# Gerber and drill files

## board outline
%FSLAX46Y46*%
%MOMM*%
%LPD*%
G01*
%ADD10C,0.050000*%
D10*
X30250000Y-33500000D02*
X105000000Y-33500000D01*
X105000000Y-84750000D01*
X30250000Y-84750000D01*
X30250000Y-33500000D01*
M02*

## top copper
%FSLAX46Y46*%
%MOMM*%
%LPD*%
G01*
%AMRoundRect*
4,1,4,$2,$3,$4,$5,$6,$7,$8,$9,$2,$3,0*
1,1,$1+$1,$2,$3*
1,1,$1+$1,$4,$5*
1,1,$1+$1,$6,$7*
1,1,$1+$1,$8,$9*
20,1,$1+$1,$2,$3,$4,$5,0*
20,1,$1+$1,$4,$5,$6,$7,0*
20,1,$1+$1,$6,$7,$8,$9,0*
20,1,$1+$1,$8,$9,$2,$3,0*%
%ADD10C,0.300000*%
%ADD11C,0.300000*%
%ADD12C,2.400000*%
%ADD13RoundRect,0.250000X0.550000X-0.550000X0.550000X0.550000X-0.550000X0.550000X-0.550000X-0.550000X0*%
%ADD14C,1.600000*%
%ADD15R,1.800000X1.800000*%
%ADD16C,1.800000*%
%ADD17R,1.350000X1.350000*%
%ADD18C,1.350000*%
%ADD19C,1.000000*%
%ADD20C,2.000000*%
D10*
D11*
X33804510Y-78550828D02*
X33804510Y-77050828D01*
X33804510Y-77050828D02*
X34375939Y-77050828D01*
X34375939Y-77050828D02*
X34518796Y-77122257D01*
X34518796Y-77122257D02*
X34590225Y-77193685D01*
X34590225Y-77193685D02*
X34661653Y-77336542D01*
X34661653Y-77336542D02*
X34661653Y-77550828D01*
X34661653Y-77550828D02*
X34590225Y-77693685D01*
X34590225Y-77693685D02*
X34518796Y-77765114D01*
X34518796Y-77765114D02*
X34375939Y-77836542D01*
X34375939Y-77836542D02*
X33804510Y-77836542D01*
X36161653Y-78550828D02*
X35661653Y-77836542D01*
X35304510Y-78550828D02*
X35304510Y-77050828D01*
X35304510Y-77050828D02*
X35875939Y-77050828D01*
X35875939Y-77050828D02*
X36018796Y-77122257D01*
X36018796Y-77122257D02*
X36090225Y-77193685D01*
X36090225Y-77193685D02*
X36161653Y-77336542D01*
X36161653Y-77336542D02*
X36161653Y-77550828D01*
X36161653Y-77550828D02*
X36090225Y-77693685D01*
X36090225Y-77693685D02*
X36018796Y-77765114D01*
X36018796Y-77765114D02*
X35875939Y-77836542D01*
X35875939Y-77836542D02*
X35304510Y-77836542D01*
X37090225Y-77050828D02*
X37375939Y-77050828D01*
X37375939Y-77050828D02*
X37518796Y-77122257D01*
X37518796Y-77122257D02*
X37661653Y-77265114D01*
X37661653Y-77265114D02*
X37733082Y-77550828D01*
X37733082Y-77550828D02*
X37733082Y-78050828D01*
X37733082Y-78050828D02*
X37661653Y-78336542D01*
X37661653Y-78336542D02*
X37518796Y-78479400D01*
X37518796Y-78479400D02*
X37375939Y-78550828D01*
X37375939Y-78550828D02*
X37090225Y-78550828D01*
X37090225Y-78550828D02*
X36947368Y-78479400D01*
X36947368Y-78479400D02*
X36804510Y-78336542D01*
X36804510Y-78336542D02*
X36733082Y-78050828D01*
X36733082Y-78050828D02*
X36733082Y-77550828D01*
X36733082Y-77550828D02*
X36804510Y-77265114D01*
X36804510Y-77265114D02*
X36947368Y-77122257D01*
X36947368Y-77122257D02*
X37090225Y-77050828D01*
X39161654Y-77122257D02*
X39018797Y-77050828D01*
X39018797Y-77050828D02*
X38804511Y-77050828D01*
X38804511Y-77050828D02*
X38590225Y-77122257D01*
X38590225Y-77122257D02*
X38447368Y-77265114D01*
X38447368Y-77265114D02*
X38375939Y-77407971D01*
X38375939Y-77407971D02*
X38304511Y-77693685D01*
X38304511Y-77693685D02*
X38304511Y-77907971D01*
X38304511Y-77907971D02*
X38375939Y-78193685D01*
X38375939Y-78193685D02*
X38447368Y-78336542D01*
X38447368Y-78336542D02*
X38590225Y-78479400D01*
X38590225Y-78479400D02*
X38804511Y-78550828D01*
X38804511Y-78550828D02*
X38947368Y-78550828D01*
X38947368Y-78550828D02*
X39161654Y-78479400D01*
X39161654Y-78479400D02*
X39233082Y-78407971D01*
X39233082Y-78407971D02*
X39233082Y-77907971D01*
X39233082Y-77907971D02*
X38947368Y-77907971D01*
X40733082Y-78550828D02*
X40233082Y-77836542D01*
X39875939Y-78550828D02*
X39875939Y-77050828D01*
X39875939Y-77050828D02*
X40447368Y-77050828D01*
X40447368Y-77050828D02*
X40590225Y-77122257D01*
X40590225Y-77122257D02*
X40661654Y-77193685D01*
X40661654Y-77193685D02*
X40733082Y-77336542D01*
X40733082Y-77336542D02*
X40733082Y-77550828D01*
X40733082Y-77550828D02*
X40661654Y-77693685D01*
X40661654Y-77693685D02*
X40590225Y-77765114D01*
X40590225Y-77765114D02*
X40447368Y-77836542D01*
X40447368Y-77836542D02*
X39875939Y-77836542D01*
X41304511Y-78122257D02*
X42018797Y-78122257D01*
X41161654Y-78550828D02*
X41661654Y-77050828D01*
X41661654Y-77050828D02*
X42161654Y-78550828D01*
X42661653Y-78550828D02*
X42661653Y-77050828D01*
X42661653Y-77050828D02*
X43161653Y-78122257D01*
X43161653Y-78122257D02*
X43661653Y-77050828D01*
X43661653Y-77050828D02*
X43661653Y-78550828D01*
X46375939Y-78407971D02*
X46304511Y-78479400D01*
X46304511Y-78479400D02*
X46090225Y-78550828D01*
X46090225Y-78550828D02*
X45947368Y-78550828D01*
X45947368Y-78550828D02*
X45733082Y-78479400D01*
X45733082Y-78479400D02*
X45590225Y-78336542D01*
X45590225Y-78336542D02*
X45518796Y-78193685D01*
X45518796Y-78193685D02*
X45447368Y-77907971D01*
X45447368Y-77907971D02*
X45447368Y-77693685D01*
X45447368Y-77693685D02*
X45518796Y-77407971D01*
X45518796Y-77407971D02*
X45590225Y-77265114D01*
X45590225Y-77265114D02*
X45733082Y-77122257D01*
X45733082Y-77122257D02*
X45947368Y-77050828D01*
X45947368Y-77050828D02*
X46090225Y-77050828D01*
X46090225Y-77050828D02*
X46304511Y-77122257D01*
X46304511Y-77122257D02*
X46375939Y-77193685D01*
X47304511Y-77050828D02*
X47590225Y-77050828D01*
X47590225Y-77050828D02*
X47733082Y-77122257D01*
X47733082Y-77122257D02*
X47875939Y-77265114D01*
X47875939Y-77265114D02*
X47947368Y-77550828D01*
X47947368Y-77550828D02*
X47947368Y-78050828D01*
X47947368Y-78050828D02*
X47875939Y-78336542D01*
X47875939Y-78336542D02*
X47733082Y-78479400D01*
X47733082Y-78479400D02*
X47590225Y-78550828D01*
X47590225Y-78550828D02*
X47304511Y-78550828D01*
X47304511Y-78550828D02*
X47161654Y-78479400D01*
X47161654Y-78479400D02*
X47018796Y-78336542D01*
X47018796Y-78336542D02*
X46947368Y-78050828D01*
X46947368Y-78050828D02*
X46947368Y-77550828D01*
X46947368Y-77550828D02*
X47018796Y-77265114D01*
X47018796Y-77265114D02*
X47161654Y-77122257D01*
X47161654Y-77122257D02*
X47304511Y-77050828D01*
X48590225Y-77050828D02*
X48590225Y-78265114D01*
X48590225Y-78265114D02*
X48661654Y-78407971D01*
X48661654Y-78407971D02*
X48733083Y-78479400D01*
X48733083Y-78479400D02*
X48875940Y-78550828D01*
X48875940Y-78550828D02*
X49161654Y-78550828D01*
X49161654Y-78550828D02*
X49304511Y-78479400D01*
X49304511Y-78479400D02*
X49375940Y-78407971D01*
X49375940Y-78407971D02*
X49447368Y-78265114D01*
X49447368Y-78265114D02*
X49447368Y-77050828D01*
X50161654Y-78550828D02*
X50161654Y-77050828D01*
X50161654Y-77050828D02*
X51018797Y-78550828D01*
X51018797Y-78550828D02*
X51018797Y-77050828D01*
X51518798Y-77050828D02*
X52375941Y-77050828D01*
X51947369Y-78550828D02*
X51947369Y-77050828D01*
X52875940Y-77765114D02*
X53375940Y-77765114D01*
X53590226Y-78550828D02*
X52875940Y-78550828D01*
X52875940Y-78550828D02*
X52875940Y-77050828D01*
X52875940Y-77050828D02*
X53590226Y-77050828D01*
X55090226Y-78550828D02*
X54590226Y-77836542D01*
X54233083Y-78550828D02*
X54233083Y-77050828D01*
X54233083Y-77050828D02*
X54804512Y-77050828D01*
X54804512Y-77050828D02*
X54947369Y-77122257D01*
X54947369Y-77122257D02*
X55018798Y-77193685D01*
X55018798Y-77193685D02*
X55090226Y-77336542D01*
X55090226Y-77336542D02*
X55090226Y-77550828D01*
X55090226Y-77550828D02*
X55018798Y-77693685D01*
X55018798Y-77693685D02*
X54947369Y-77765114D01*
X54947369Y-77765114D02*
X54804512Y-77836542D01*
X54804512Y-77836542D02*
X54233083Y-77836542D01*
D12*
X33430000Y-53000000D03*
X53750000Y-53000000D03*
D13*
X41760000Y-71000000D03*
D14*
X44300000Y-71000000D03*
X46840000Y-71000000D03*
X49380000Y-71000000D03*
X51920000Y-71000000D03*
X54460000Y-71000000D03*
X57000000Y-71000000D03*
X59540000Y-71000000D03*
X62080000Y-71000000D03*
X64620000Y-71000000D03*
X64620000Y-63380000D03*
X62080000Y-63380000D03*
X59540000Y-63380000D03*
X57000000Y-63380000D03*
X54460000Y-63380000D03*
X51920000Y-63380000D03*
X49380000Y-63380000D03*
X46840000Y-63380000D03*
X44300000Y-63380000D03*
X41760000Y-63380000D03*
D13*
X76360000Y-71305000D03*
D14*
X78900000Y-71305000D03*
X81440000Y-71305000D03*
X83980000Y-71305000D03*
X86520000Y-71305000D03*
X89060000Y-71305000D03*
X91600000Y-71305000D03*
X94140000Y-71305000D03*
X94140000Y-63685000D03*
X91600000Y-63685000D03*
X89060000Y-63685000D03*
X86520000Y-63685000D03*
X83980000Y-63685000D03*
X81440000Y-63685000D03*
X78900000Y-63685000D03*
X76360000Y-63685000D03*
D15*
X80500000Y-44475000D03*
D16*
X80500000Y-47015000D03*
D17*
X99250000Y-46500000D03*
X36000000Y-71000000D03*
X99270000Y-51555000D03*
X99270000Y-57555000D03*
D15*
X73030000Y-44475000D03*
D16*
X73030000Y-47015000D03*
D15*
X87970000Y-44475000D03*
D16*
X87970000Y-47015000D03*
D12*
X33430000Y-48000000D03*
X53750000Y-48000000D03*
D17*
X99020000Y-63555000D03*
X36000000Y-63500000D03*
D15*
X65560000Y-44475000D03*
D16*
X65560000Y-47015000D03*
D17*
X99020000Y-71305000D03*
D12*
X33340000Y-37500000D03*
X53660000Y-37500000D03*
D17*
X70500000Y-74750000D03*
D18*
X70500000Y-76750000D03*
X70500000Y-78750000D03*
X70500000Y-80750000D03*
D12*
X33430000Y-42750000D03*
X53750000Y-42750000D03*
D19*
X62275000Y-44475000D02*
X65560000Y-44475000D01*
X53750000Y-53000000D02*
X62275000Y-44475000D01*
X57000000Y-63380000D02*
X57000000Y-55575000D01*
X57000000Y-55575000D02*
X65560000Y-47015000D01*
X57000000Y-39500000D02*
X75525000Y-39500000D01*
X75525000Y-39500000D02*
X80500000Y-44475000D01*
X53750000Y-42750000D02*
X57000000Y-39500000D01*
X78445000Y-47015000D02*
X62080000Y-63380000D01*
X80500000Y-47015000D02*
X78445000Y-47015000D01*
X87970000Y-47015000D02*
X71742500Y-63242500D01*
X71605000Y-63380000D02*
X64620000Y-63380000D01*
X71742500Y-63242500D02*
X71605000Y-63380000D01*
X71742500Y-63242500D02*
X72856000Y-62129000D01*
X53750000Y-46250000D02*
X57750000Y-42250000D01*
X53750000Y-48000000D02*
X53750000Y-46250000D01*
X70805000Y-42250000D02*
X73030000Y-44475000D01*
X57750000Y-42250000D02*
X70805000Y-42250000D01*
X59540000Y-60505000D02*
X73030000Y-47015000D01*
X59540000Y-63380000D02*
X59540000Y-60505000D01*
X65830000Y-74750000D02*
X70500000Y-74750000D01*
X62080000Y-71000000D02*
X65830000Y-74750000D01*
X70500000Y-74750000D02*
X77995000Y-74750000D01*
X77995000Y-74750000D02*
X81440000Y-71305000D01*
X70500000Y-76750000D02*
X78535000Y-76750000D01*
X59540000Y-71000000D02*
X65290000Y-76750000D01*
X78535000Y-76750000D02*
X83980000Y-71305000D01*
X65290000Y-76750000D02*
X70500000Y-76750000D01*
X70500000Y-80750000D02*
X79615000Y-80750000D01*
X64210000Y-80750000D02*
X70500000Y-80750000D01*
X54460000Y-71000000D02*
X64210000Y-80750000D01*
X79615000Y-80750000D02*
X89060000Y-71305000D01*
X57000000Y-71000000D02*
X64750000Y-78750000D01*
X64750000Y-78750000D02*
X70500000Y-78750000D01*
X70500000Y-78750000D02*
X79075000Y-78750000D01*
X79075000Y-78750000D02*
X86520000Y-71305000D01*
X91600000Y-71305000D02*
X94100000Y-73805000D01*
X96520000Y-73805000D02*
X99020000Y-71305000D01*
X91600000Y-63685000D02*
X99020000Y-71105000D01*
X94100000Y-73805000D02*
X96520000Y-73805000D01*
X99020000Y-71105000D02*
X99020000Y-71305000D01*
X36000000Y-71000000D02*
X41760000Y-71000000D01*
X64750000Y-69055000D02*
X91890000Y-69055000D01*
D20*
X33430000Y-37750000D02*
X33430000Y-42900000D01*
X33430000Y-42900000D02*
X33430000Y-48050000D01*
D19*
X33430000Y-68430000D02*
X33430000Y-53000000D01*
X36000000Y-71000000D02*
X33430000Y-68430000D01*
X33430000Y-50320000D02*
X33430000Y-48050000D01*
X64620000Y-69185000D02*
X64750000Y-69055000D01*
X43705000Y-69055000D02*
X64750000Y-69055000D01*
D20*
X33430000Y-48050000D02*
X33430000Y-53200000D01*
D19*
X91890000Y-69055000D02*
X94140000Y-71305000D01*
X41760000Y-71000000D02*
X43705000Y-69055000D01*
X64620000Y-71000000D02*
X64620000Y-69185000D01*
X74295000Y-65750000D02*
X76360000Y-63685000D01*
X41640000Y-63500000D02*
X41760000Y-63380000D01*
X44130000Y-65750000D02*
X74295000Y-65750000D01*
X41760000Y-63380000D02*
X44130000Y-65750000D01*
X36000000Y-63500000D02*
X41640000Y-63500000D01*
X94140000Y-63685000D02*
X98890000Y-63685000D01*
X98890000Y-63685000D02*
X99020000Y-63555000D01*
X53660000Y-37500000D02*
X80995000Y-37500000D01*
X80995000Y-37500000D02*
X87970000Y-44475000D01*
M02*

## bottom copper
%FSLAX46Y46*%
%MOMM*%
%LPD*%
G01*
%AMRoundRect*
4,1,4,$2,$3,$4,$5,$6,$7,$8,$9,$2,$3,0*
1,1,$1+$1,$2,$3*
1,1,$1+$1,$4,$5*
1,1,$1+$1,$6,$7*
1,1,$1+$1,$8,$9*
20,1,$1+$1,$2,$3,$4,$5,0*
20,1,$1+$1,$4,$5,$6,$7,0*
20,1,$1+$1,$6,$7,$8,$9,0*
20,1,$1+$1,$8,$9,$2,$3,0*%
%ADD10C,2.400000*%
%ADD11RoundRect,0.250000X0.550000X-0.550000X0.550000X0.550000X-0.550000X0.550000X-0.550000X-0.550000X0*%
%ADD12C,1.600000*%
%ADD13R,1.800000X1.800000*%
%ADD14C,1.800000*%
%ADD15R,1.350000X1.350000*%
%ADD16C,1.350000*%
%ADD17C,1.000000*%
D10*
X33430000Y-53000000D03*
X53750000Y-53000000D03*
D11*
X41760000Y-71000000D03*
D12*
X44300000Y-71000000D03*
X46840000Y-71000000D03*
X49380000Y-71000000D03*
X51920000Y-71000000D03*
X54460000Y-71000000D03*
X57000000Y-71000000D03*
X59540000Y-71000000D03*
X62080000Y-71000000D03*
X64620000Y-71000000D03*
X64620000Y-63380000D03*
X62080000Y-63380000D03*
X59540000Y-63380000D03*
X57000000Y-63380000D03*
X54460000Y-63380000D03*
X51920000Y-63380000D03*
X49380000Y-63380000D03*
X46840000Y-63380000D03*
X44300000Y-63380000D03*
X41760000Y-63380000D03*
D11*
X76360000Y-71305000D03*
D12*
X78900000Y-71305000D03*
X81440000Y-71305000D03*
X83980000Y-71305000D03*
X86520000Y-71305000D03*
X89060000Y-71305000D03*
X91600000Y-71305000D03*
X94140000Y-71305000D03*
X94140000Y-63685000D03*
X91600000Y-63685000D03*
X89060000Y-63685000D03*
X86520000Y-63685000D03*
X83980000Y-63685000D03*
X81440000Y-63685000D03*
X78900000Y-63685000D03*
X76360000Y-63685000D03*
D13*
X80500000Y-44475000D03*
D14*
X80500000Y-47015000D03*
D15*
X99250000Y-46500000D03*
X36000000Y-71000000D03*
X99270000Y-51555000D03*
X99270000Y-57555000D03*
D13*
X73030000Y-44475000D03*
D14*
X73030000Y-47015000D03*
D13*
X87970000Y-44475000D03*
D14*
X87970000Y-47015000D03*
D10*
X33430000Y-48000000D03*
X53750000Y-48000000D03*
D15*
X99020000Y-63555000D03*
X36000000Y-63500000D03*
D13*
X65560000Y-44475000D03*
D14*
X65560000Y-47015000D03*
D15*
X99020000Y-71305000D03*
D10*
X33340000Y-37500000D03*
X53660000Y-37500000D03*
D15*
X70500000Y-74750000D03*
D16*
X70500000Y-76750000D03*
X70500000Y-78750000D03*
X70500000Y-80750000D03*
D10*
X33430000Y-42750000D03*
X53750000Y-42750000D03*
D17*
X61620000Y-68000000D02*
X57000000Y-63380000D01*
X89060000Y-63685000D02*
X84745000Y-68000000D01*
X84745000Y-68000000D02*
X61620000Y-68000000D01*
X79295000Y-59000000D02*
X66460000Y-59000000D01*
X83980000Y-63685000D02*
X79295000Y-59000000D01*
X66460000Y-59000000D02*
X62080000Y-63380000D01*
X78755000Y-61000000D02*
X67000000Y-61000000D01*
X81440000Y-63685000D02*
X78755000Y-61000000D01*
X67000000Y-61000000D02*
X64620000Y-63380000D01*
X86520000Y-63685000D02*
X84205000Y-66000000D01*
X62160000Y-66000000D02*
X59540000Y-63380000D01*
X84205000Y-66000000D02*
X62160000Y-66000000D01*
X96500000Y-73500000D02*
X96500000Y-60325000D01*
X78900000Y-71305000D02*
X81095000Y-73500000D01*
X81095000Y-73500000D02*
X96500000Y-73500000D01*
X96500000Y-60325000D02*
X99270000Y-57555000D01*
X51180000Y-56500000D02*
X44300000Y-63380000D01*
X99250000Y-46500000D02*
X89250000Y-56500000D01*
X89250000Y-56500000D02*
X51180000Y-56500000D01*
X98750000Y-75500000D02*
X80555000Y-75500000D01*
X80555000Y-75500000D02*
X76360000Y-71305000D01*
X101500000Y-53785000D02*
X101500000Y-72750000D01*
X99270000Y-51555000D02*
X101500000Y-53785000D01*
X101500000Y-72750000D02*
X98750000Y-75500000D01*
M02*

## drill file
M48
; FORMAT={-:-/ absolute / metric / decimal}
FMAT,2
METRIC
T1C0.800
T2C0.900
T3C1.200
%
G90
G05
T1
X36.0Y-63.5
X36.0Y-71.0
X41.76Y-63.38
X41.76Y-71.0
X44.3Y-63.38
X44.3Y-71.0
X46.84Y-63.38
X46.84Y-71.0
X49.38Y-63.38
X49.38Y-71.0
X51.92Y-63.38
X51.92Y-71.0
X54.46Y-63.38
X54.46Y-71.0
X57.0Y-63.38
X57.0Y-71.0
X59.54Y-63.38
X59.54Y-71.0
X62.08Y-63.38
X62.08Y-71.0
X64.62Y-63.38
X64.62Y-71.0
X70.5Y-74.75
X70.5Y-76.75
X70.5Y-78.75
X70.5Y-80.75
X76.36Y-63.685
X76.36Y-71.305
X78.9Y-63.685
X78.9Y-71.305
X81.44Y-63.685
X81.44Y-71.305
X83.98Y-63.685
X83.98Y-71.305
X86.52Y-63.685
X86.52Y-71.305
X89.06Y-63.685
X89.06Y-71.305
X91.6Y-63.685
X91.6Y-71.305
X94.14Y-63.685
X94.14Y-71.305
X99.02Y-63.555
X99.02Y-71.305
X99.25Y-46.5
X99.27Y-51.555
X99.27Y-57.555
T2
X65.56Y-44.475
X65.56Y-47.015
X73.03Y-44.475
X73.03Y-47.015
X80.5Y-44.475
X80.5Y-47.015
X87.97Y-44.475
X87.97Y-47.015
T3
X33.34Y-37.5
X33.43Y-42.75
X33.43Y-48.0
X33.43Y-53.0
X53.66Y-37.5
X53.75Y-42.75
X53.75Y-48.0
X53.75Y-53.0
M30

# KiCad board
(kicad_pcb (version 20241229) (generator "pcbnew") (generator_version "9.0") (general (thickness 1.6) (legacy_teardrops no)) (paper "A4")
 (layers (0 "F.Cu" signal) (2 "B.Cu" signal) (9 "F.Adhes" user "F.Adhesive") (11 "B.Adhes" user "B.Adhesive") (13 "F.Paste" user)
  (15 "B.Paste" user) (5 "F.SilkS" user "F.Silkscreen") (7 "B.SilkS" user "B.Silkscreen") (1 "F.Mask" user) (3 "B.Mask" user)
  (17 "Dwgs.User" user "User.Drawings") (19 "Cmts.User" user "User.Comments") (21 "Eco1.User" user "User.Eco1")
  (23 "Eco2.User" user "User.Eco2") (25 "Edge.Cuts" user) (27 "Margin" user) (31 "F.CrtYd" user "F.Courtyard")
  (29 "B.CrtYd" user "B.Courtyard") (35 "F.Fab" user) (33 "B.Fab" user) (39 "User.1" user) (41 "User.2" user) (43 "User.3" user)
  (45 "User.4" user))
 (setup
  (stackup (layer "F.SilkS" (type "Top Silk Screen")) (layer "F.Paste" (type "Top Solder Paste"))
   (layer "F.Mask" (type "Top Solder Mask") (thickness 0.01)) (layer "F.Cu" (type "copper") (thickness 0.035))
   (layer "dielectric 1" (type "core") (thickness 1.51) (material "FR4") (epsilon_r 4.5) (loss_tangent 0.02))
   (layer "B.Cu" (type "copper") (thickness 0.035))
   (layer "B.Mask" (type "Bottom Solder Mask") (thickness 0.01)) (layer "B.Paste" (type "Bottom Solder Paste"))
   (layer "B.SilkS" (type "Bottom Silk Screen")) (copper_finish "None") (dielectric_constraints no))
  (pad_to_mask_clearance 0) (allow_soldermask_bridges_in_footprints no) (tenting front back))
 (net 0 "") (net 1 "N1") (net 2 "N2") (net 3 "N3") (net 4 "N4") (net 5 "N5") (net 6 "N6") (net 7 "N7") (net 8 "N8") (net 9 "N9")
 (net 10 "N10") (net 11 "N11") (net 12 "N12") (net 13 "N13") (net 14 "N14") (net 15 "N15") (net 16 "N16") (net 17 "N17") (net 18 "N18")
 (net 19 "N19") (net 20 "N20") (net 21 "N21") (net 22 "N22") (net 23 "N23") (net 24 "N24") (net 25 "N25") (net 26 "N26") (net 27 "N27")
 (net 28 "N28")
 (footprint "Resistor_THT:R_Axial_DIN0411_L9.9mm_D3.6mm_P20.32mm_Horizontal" (layer "F.Cu") (at 33.43 53)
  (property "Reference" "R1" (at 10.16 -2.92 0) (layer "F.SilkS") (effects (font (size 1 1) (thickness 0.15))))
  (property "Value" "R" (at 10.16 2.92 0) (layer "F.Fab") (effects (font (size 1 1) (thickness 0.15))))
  (pad "1" thru_hole circle (at 0 0) (size 2.4 2.4) (drill 1.2) (layers "*.Cu" "*.Mask") (remove_unused_layers no) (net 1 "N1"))
  (pad "2" thru_hole circle (at 20.32 0) (size 2.4 2.4) (drill 1.2) (layers "*.Cu" "*.Mask") (remove_unused_layers no) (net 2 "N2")))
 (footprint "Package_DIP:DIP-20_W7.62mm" (layer "F.Cu") (at 41.76 71 90)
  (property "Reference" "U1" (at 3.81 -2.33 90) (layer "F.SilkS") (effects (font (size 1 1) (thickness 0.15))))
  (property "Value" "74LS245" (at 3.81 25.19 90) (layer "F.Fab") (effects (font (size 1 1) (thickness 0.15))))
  (pad "1" thru_hole roundrect (at 0 0 90) (size 1.6 1.6) (drill 0.8) (layers "*.Cu" "*.Mask") (remove_unused_layers no)
   (roundrect_rratio 0.15625) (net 1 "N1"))
  (pad "2" thru_hole circle (at 0 2.54 90) (size 1.6 1.6) (drill 0.8) (layers "*.Cu" "*.Mask") (remove_unused_layers no) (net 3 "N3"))
  (pad "3" thru_hole circle (at 0 5.08 90) (size 1.6 1.6) (drill 0.8) (layers "*.Cu" "*.Mask") (remove_unused_layers no) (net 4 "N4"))
  (pad "4" thru_hole circle (at 0 7.62 90) (size 1.6 1.6) (drill 0.8) (layers "*.Cu" "*.Mask") (remove_unused_layers no) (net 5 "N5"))
  (pad "5" thru_hole circle (at 0 10.16 90) (size 1.6 1.6) (drill 0.8) (layers "*.Cu" "*.Mask") (remove_unused_layers no) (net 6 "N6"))
  (pad "6" thru_hole circle (at 0 12.7 90) (size 1.6 1.6) (drill 0.8) (layers "*.Cu" "*.Mask") (remove_unused_layers no) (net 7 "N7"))
  (pad "7" thru_hole circle (at 0 15.24 90) (size 1.6 1.6) (drill 0.8) (layers "*.Cu" "*.Mask") (remove_unused_layers no) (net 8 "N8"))
  (pad "8" thru_hole circle (at 0 17.78 90) (size 1.6 1.6) (drill 0.8) (layers "*.Cu" "*.Mask") (remove_unused_layers no) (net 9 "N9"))
  (pad "9" thru_hole circle (at 0 20.32 90) (size 1.6 1.6) (drill 0.8) (layers "*.Cu" "*.Mask") (remove_unused_layers no) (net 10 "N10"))
  (pad "10" thru_hole circle (at 0 22.86 90) (size 1.6 1.6) (drill 0.8) (layers "*.Cu" "*.Mask") (remove_unused_layers no) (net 1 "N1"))
  (pad "11" thru_hole circle (at 7.62 22.86 90) (size 1.6 1.6) (drill 0.8) (layers "*.Cu" "*.Mask") (remove_unused_layers no) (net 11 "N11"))
  (pad "12" thru_hole circle (at 7.62 20.32 90) (size 1.6 1.6) (drill 0.8) (layers "*.Cu" "*.Mask") (remove_unused_layers no) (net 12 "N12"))
  (pad "13" thru_hole circle (at 7.62 17.78 90) (size 1.6 1.6) (drill 0.8) (layers "*.Cu" "*.Mask") (remove_unused_layers no) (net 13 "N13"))
  (pad "14" thru_hole circle (at 7.62 15.24 90) (size 1.6 1.6) (drill 0.8) (layers "*.Cu" "*.Mask") (remove_unused_layers no) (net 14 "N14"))
  (pad "15" thru_hole circle (at 7.62 12.7 90) (size 1.6 1.6) (drill 0.8) (layers "*.Cu" "*.Mask") (remove_unused_layers no) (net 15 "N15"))
  (pad "16" thru_hole circle (at 7.62 10.16 90) (size 1.6 1.6) (drill 0.8) (layers "*.Cu" "*.Mask") (remove_unused_layers no) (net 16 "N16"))
  (pad "17" thru_hole circle (at 7.62 7.62 90) (size 1.6 1.6) (drill 0.8) (layers "*.Cu" "*.Mask") (remove_unused_layers no) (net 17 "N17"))
  (pad "18" thru_hole circle (at 7.62 5.08 90) (size 1.6 1.6) (drill 0.8) (layers "*.Cu" "*.Mask") (remove_unused_layers no) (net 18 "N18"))
  (pad "19" thru_hole circle (at 7.62 2.54 90) (size 1.6 1.6) (drill 0.8) (layers "*.Cu" "*.Mask") (remove_unused_layers no) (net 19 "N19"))
  (pad "20" thru_hole circle (at 7.62 0 90) (size 1.6 1.6) (drill 0.8) (layers "*.Cu" "*.Mask") (remove_unused_layers no) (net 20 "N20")))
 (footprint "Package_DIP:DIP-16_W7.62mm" (layer "F.Cu") (at 76.36 71.305 90)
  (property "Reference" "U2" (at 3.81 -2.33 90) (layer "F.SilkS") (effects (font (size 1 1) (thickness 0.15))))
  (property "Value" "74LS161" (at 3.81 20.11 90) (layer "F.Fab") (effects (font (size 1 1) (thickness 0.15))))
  (pad "1" thru_hole roundrect (at 0 0 90) (size 1.6 1.6) (drill 0.8) (layers "*.Cu" "*.Mask") (remove_unused_layers no)
   (roundrect_rratio 0.15625) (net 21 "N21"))
  (pad "2" thru_hole circle (at 0 2.54 90) (size 1.6 1.6) (drill 0.8) (layers "*.Cu" "*.Mask") (remove_unused_layers no) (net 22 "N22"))
  (pad "3" thru_hole circle (at 0 5.08 90) (size 1.6 1.6) (drill 0.8) (layers "*.Cu" "*.Mask") (remove_unused_layers no) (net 10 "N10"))
  (pad "4" thru_hole circle (at 0 7.62 90) (size 1.6 1.6) (drill 0.8) (layers "*.Cu" "*.Mask") (remove_unused_layers no) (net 9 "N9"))
  (pad "5" thru_hole circle (at 0 10.16 90) (size 1.6 1.6) (drill 0.8) (layers "*.Cu" "*.Mask") (remove_unused_layers no) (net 8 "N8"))
  (pad "6" thru_hole circle (at 0 12.7 90) (size 1.6 1.6) (drill 0.8) (layers "*.Cu" "*.Mask") (remove_unused_layers no) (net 7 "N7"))
  (pad "7" thru_hole circle (at 0 15.24 90) (size 1.6 1.6) (drill 0.8) (layers "*.Cu" "*.Mask") (remove_unused_layers no) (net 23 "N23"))
  (pad "8" thru_hole circle (at 0 17.78 90) (size 1.6 1.6) (drill 0.8) (layers "*.Cu" "*.Mask") (remove_unused_layers no) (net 1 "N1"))
  (pad "9" thru_hole circle (at 7.62 17.78 90) (size 1.6 1.6) (drill 0.8) (layers "*.Cu" "*.Mask") (remove_unused_layers no) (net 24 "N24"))
  (pad "10" thru_hole circle (at 7.62 15.24 90) (size 1.6 1.6) (drill 0.8) (layers "*.Cu" "*.Mask") (remove_unused_layers no) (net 23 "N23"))
  (pad "11" thru_hole circle (at 7.62 12.7 90) (size 1.6 1.6) (drill 0.8) (layers "*.Cu" "*.Mask") (remove_unused_layers no) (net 14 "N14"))
  (pad "12" thru_hole circle (at 7.62 10.16 90) (size 1.6 1.6) (drill 0.8) (layers "*.Cu" "*.Mask") (remove_unused_layers no) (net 13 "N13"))
  (pad "13" thru_hole circle (at 7.62 7.62 90) (size 1.6 1.6) (drill 0.8) (layers "*.Cu" "*.Mask") (remove_unused_layers no) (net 12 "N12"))
  (pad "14" thru_hole circle (at 7.62 5.08 90) (size 1.6 1.6) (drill 0.8) (layers "*.Cu" "*.Mask") (remove_unused_layers no) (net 11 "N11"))
  (pad "15" thru_hole circle (at 7.62 2.54 90) (size 1.6 1.6) (drill 0.8) (layers "*.Cu" "*.Mask") (remove_unused_layers no) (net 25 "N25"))
  (pad "16" thru_hole circle (at 7.62 0 90) (size 1.6 1.6) (drill 0.8) (layers "*.Cu" "*.Mask") (remove_unused_layers no) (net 20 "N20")))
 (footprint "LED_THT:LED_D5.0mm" (layer "F.Cu") (at 80.5 44.475 -90)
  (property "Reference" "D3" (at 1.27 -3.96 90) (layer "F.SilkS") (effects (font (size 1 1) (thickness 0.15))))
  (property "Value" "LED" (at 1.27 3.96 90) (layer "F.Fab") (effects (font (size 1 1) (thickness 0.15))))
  (pad "1" thru_hole rect (at 0 0 270) (size 1.8 1.8) (drill 0.9) (layers "*.Cu" "*.Mask") (remove_unused_layers no) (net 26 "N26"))
  (pad "2" thru_hole circle (at 2.54 0 270) (size 1.8 1.8) (drill 0.9) (layers "*.Cu" "*.Mask") (remove_unused_layers no) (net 12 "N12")))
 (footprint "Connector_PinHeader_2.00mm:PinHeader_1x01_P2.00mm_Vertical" (layer "F.Cu") (at 99.25 46.5)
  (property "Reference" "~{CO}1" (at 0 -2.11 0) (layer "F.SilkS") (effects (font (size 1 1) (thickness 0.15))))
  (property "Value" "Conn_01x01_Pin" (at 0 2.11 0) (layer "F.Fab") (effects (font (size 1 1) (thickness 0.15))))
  (pad "1" thru_hole rect (at 0 0) (size 1.35 1.35) (drill 0.8) (layers "*.Cu" "*.Mask") (remove_unused_layers no) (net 19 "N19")))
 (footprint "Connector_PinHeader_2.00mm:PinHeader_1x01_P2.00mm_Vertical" (layer "F.Cu") (at 36 71)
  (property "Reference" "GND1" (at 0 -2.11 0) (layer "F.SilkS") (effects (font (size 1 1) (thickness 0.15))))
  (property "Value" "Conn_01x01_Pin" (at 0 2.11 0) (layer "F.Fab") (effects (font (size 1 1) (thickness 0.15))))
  (pad "1" thru_hole rect (at 0 0) (size 1.35 1.35) (drill 0.8) (layers "*.Cu" "*.Mask") (remove_unused_layers no) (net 1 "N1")))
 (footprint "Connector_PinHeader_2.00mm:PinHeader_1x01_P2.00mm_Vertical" (layer "F.Cu") (at 99.27 51.555)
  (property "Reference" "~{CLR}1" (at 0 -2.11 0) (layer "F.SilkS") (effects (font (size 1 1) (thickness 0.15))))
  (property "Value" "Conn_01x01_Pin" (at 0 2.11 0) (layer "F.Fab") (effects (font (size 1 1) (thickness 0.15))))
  (pad "1" thru_hole rect (at 0 0) (size 1.35 1.35) (drill 0.8) (layers "*.Cu" "*.Mask") (remove_unused_layers no) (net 21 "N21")))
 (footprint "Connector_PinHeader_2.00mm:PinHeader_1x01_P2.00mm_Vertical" (layer "F.Cu") (at 99.27 57.555)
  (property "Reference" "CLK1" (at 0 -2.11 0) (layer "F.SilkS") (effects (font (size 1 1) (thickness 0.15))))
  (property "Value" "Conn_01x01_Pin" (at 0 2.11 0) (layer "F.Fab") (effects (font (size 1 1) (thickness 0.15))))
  (pad "1" thru_hole rect (at 0 0) (size 1.35 1.35) (drill 0.8) (layers "*.Cu" "*.Mask") (remove_unused_layers no) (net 22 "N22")))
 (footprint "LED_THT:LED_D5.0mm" (layer "F.Cu") (at 73.03 44.475 -90)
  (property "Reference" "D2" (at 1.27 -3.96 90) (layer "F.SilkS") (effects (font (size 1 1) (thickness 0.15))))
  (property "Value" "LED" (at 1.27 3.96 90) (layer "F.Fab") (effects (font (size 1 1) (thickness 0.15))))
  (pad "1" thru_hole rect (at 0 0 270) (size 1.8 1.8) (drill 0.9) (layers "*.Cu" "*.Mask") (remove_unused_layers no) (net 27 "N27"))
  (pad "2" thru_hole circle (at 2.54 0 270) (size 1.8 1.8) (drill 0.9) (layers "*.Cu" "*.Mask") (remove_unused_layers no) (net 13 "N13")))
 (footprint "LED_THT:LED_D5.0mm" (layer "F.Cu") (at 87.97 44.475 -90)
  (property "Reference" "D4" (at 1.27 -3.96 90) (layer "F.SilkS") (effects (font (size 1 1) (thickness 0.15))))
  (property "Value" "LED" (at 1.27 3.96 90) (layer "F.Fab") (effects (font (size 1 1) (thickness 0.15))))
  (pad "1" thru_hole rect (at 0 0 270) (size 1.8 1.8) (drill 0.9) (layers "*.Cu" "*.Mask") (remove_unused_layers no) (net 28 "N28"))
  (pad "2" thru_hole circle (at 2.54 0 270) (size 1.8 1.8) (drill 0.9) (layers "*.Cu" "*.Mask") (remove_unused_layers no) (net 11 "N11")))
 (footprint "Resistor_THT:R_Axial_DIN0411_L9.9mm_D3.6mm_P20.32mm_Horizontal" (layer "F.Cu") (at 33.43 48)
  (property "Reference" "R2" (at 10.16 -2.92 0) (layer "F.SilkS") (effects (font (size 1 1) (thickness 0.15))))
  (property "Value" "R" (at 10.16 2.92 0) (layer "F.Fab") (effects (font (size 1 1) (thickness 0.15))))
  (pad "1" thru_hole circle (at 0 0) (size 2.4 2.4) (drill 1.2) (layers "*.Cu" "*.Mask") (remove_unused_layers no) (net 1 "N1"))
  (pad "2" thru_hole circle (at 20.32 0) (size 2.4 2.4) (drill 1.2) (layers "*.Cu" "*.Mask") (remove_unused_layers no) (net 27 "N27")))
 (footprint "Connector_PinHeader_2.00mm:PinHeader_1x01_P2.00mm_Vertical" (layer "F.Cu") (at 99.02 63.555)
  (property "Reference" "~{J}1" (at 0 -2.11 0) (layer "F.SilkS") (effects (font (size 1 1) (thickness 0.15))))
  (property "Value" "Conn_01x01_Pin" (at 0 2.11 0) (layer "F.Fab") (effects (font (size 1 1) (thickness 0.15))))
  (pad "1" thru_hole rect (at 0 0) (size 1.35 1.35) (drill 0.8) (layers "*.Cu" "*.Mask") (remove_unused_layers no) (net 24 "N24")))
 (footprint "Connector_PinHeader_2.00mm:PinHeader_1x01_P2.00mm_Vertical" (layer "F.Cu") (at 36 63.5)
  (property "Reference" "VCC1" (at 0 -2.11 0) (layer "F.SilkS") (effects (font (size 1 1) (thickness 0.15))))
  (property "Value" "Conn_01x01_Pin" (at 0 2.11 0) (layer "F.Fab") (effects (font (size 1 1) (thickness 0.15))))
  (pad "1" thru_hole rect (at 0 0) (size 1.35 1.35) (drill 0.8) (layers "*.Cu" "*.Mask") (remove_unused_layers no) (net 20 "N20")))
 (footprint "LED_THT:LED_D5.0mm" (layer "F.Cu") (at 65.56 44.475 -90)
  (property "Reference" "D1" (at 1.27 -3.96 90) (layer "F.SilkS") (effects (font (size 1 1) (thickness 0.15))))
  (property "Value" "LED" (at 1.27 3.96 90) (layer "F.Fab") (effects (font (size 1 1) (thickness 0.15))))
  (pad "1" thru_hole rect (at 0 0 270) (size 1.8 1.8) (drill 0.9) (layers "*.Cu" "*.Mask") (remove_unused_layers no) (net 2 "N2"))
  (pad "2" thru_hole circle (at 2.54 0 270) (size 1.8 1.8) (drill 0.9) (layers "*.Cu" "*.Mask") (remove_unused_layers no) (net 14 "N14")))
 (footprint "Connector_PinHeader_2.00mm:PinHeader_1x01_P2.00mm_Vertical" (layer "F.Cu") (at 99.02 71.305)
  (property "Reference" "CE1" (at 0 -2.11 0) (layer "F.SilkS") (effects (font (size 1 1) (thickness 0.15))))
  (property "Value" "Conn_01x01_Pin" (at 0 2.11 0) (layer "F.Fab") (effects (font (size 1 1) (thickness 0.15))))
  (pad "1" thru_hole rect (at 0 0) (size 1.35 1.35) (drill 0.8) (layers "*.Cu" "*.Mask") (remove_unused_layers no) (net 23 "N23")))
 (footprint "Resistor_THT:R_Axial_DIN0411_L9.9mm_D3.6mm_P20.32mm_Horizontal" (layer "F.Cu") (at 33.34 37.5)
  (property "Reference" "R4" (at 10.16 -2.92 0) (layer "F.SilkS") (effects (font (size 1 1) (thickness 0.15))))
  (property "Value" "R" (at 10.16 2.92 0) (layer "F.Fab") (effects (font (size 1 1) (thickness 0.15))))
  (pad "1" thru_hole circle (at 0 0) (size 2.4 2.4) (drill 1.2) (layers "*.Cu" "*.Mask") (remove_unused_layers no) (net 1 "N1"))
  (pad "2" thru_hole circle (at 20.32 0) (size 2.4 2.4) (drill 1.2) (layers "*.Cu" "*.Mask") (remove_unused_layers no) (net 28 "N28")))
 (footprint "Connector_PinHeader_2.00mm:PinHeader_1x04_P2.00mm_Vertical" (layer "F.Cu") (at 70.5 74.75)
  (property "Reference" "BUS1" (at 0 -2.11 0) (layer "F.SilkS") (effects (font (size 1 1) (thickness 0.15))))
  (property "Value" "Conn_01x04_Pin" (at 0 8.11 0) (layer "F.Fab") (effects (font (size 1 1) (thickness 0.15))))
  (pad "1" thru_hole rect (at 0 0) (size 1.35 1.35) (drill 0.8) (layers "*.Cu" "*.Mask") (remove_unused_layers no) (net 10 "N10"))
  (pad "2" thru_hole circle (at 0 2) (size 1.35 1.35) (drill 0.8) (layers "*.Cu" "*.Mask") (remove_unused_layers no) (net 9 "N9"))
  (pad "3" thru_hole circle (at 0 4) (size 1.35 1.35) (drill 0.8) (layers "*.Cu" "*.Mask") (remove_unused_layers no) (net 8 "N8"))
  (pad "4" thru_hole circle (at 0 6) (size 1.35 1.35) (drill 0.8) (layers "*.Cu" "*.Mask") (remove_unused_layers no) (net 7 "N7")))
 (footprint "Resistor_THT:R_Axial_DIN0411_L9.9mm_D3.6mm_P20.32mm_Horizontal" (layer "F.Cu") (at 33.43 42.75)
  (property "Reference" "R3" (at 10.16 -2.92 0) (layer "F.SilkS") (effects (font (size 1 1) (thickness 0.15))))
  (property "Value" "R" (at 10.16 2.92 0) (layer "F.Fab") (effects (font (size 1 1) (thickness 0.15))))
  (pad "1" thru_hole circle (at 0 0) (size 2.4 2.4) (drill 1.2) (layers "*.Cu" "*.Mask") (remove_unused_layers no) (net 1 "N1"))
  (pad "2" thru_hole circle (at 20.32 0) (size 2.4 2.4) (drill 1.2) (layers "*.Cu" "*.Mask") (remove_unused_layers no) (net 26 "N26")))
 (gr_rect (start 30.25 33.5) (end 105 84.75) (stroke (width 0.05) (type default)) (fill no) (layer "Edge.Cuts"))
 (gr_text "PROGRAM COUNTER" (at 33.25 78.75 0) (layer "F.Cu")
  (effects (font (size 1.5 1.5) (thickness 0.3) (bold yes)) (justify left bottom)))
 (segment (start 62.275 44.475) (end 65.56 44.475) (width 1) (layer "F.Cu") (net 2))
 (segment (start 53.75 53) (end 62.275 44.475) (width 1) (layer "F.Cu") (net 2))
 (segment (start 57 63.38) (end 57 55.575) (width 1) (layer "F.Cu") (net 14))
 (segment (start 57 55.575) (end 65.56 47.015) (width 1) (layer "F.Cu") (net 14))
 (segment (start 61.62 68) (end 57 63.38) (width 1) (layer "B.Cu") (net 14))
 (segment (start 89.06 63.685) (end 84.745 68) (width 1) (layer "B.Cu") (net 14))
 (segment (start 84.745 68) (end 61.62 68) (width 1) (layer "B.Cu") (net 14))
 (segment (start 57 39.5) (end 75.525 39.5) (width 1) (layer "F.Cu") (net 26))
 (segment (start 75.525 39.5) (end 80.5 44.475) (width 1) (layer "F.Cu") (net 26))
 (segment (start 53.75 42.75) (end 57 39.5) (width 1) (layer "F.Cu") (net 26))
 (segment (start 78.445 47.015) (end 62.08 63.38) (width 1) (layer "F.Cu") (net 12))
 (segment (start 80.5 47.015) (end 78.445 47.015) (width 1) (layer "F.Cu") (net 12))
 (segment (start 79.295 59) (end 66.46 59) (width 1) (layer "B.Cu") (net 12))
 (segment (start 83.98 63.685) (end 79.295 59) (width 1) (layer "B.Cu") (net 12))
 (segment (start 66.46 59) (end 62.08 63.38) (width 1) (layer "B.Cu") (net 12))
 (segment (start 87.97 47.015) (end 71.7425 63.2425) (width 1) (layer "F.Cu") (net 11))
 (segment (start 71.605 63.38) (end 64.62 63.38) (width 1) (layer "F.Cu") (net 11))
 (segment (start 71.7425 63.2425) (end 71.605 63.38) (width 1) (layer "F.Cu") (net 11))
 (segment (start 71.7425 63.2425) (end 72.856 62.129) (width 1) (layer "F.Cu") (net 11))
 (segment (start 78.755 61) (end 67 61) (width 1) (layer "B.Cu") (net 11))
 (segment (start 81.44 63.685) (end 78.755 61) (width 1) (layer "B.Cu") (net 11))
 (segment (start 67 61) (end 64.62 63.38) (width 1) (layer "B.Cu") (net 11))
 (segment (start 53.75 46.25) (end 57.75 42.25) (width 1) (layer "F.Cu") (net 27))
 (segment (start 53.75 48) (end 53.75 46.25) (width 1) (layer "F.Cu") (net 27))
 (segment (start 70.805 42.25) (end 73.03 44.475) (width 1) (layer "F.Cu") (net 27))
 (segment (start 57.75 42.25) (end 70.805 42.25) (width 1) (layer "F.Cu") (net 27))
 (segment (start 59.54 60.505) (end 73.03 47.015) (width 1) (layer "F.Cu") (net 13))
 (segment (start 59.54 63.38) (end 59.54 60.505) (width 1) (layer "F.Cu") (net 13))
 (segment (start 86.52 63.685) (end 84.205 66) (width 1) (layer "B.Cu") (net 13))
 (segment (start 62.16 66) (end 59.54 63.38) (width 1) (layer "B.Cu") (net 13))
 (segment (start 84.205 66) (end 62.16 66) (width 1) (layer "B.Cu") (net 13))
 (segment (start 65.83 74.75) (end 70.5 74.75) (width 1) (layer "F.Cu") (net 10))
 (segment (start 62.08 71) (end 65.83 74.75) (width 1) (layer "F.Cu") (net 10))
 (segment (start 70.5 74.75) (end 77.995 74.75) (width 1) (layer "F.Cu") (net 10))
 (segment (start 77.995 74.75) (end 81.44 71.305) (width 1) (layer "F.Cu") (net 10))
 (segment (start 70.5 76.75) (end 78.535 76.75) (width 1) (layer "F.Cu") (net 9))
 (segment (start 59.54 71) (end 65.29 76.75) (width 1) (layer "F.Cu") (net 9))
 (segment (start 78.535 76.75) (end 83.98 71.305) (width 1) (layer "F.Cu") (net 9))
 (segment (start 65.29 76.75) (end 70.5 76.75) (width 1) (layer "F.Cu") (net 9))
 (segment (start 70.5 80.75) (end 79.615 80.75) (width 1) (layer "F.Cu") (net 7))
 (segment (start 64.21 80.75) (end 70.5 80.75) (width 1) (layer "F.Cu") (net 7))
 (segment (start 54.46 71) (end 64.21 80.75) (width 1) (layer "F.Cu") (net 7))
 (segment (start 79.615 80.75) (end 89.06 71.305) (width 1) (layer "F.Cu") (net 7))
 (segment (start 57 71) (end 64.75 78.75) (width 1) (layer "F.Cu") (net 8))
 (segment (start 64.75 78.75) (end 70.5 78.75) (width 1) (layer "F.Cu") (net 8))
 (segment (start 70.5 78.75) (end 79.075 78.75) (width 1) (layer "F.Cu") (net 8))
 (segment (start 79.075 78.75) (end 86.52 71.305) (width 1) (layer "F.Cu") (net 8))
 (segment (start 91.6 71.305) (end 94.1 73.805) (width 1) (layer "F.Cu") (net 23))
 (segment (start 96.52 73.805) (end 99.02 71.305) (width 1) (layer "F.Cu") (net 23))
 (segment (start 91.6 63.685) (end 99.02 71.105) (width 1) (layer "F.Cu") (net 23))
 (segment (start 94.1 73.805) (end 96.52 73.805) (width 1) (layer "F.Cu") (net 23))
 (segment (start 99.02 71.105) (end 99.02 71.305) (width 1) (layer "F.Cu") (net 23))
 (segment (start 96.5 73.5) (end 96.5 60.325) (width 1) (layer "B.Cu") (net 22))
 (segment (start 78.9 71.305) (end 81.095 73.5) (width 1) (layer "B.Cu") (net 22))
 (segment (start 81.095 73.5) (end 96.5 73.5) (width 1) (layer "B.Cu") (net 22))
 (segment (start 96.5 60.325) (end 99.27 57.555) (width 1) (layer "B.Cu") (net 22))
 (segment (start 36 71) (end 41.76 71) (width 1) (layer "F.Cu") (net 1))
 (segment (start 64.75 69.055) (end 91.89 69.055) (width 1) (layer "F.Cu") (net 1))
 (segment (start 33.43 37.75) (end 33.43 42.9) (width 2) (layer "F.Cu") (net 1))
 (segment (start 33.43 42.9) (end 33.43 48.05) (width 2) (layer "F.Cu") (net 1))
 (segment (start 33.43 68.43) (end 33.43 53) (width 1) (layer "F.Cu") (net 1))
 (segment (start 36 71) (end 33.43 68.43) (width 1) (layer "F.Cu") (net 1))
 (segment (start 33.43 50.32) (end 33.43 48.05) (width 1) (layer "F.Cu") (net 1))
 (segment (start 64.62 69.185) (end 64.75 69.055) (width 1) (layer "F.Cu") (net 1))
 (segment (start 43.705 69.055) (end 64.75 69.055) (width 1) (layer "F.Cu") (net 1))
 (segment (start 33.43 48.05) (end 33.43 53.2) (width 2) (layer "F.Cu") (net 1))
 (segment (start 91.89 69.055) (end 94.14 71.305) (width 1) (layer "F.Cu") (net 1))
 (segment (start 41.76 71) (end 43.705 69.055) (width 1) (layer "F.Cu") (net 1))
 (segment (start 64.62 71) (end 64.62 69.185) (width 1) (layer "F.Cu") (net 1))
 (segment (start 74.295 65.75) (end 76.36 63.685) (width 1) (layer "F.Cu") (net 20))
 (segment (start 41.64 63.5) (end 41.76 63.38) (width 1) (layer "F.Cu") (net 20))
 (segment (start 44.13 65.75) (end 74.295 65.75) (width 1) (layer "F.Cu") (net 20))
 (segment (start 41.76 63.38) (end 44.13 65.75) (width 1) (layer "F.Cu") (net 20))
 (segment (start 36 63.5) (end 41.64 63.5) (width 1) (layer "F.Cu") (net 20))
 (segment (start 51.18 56.5) (end 44.3 63.38) (width 1) (layer "B.Cu") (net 19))
 (segment (start 99.25 46.5) (end 89.25 56.5) (width 1) (layer "B.Cu") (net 19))
 (segment (start 89.25 56.5) (end 51.18 56.5) (width 1) (layer "B.Cu") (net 19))
 (segment (start 98.75 75.5) (end 80.555 75.5) (width 1) (layer "B.Cu") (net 21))
 (segment (start 80.555 75.5) (end 76.36 71.305) (width 1) (layer "B.Cu") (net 21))
 (segment (start 101.5 53.785) (end 101.5 72.75) (width 1) (layer "B.Cu") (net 21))
 (segment (start 99.27 51.555) (end 101.5 53.785) (width 1) (layer "B.Cu") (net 21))
 (segment (start 101.5 72.75) (end 98.75 75.5) (width 1) (layer "B.Cu") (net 21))
 (segment (start 94.14 63.685) (end 98.89 63.685) (width 1) (layer "F.Cu") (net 24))
 (segment (start 98.89 63.685) (end 99.02 63.555) (width 1) (layer "F.Cu") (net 24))
 (segment (start 53.66 37.5) (end 80.995 37.5) (width 1) (layer "F.Cu") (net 28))
 (segment (start 80.995 37.5) (end 87.97 44.475) (width 1) (layer "F.Cu") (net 28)))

